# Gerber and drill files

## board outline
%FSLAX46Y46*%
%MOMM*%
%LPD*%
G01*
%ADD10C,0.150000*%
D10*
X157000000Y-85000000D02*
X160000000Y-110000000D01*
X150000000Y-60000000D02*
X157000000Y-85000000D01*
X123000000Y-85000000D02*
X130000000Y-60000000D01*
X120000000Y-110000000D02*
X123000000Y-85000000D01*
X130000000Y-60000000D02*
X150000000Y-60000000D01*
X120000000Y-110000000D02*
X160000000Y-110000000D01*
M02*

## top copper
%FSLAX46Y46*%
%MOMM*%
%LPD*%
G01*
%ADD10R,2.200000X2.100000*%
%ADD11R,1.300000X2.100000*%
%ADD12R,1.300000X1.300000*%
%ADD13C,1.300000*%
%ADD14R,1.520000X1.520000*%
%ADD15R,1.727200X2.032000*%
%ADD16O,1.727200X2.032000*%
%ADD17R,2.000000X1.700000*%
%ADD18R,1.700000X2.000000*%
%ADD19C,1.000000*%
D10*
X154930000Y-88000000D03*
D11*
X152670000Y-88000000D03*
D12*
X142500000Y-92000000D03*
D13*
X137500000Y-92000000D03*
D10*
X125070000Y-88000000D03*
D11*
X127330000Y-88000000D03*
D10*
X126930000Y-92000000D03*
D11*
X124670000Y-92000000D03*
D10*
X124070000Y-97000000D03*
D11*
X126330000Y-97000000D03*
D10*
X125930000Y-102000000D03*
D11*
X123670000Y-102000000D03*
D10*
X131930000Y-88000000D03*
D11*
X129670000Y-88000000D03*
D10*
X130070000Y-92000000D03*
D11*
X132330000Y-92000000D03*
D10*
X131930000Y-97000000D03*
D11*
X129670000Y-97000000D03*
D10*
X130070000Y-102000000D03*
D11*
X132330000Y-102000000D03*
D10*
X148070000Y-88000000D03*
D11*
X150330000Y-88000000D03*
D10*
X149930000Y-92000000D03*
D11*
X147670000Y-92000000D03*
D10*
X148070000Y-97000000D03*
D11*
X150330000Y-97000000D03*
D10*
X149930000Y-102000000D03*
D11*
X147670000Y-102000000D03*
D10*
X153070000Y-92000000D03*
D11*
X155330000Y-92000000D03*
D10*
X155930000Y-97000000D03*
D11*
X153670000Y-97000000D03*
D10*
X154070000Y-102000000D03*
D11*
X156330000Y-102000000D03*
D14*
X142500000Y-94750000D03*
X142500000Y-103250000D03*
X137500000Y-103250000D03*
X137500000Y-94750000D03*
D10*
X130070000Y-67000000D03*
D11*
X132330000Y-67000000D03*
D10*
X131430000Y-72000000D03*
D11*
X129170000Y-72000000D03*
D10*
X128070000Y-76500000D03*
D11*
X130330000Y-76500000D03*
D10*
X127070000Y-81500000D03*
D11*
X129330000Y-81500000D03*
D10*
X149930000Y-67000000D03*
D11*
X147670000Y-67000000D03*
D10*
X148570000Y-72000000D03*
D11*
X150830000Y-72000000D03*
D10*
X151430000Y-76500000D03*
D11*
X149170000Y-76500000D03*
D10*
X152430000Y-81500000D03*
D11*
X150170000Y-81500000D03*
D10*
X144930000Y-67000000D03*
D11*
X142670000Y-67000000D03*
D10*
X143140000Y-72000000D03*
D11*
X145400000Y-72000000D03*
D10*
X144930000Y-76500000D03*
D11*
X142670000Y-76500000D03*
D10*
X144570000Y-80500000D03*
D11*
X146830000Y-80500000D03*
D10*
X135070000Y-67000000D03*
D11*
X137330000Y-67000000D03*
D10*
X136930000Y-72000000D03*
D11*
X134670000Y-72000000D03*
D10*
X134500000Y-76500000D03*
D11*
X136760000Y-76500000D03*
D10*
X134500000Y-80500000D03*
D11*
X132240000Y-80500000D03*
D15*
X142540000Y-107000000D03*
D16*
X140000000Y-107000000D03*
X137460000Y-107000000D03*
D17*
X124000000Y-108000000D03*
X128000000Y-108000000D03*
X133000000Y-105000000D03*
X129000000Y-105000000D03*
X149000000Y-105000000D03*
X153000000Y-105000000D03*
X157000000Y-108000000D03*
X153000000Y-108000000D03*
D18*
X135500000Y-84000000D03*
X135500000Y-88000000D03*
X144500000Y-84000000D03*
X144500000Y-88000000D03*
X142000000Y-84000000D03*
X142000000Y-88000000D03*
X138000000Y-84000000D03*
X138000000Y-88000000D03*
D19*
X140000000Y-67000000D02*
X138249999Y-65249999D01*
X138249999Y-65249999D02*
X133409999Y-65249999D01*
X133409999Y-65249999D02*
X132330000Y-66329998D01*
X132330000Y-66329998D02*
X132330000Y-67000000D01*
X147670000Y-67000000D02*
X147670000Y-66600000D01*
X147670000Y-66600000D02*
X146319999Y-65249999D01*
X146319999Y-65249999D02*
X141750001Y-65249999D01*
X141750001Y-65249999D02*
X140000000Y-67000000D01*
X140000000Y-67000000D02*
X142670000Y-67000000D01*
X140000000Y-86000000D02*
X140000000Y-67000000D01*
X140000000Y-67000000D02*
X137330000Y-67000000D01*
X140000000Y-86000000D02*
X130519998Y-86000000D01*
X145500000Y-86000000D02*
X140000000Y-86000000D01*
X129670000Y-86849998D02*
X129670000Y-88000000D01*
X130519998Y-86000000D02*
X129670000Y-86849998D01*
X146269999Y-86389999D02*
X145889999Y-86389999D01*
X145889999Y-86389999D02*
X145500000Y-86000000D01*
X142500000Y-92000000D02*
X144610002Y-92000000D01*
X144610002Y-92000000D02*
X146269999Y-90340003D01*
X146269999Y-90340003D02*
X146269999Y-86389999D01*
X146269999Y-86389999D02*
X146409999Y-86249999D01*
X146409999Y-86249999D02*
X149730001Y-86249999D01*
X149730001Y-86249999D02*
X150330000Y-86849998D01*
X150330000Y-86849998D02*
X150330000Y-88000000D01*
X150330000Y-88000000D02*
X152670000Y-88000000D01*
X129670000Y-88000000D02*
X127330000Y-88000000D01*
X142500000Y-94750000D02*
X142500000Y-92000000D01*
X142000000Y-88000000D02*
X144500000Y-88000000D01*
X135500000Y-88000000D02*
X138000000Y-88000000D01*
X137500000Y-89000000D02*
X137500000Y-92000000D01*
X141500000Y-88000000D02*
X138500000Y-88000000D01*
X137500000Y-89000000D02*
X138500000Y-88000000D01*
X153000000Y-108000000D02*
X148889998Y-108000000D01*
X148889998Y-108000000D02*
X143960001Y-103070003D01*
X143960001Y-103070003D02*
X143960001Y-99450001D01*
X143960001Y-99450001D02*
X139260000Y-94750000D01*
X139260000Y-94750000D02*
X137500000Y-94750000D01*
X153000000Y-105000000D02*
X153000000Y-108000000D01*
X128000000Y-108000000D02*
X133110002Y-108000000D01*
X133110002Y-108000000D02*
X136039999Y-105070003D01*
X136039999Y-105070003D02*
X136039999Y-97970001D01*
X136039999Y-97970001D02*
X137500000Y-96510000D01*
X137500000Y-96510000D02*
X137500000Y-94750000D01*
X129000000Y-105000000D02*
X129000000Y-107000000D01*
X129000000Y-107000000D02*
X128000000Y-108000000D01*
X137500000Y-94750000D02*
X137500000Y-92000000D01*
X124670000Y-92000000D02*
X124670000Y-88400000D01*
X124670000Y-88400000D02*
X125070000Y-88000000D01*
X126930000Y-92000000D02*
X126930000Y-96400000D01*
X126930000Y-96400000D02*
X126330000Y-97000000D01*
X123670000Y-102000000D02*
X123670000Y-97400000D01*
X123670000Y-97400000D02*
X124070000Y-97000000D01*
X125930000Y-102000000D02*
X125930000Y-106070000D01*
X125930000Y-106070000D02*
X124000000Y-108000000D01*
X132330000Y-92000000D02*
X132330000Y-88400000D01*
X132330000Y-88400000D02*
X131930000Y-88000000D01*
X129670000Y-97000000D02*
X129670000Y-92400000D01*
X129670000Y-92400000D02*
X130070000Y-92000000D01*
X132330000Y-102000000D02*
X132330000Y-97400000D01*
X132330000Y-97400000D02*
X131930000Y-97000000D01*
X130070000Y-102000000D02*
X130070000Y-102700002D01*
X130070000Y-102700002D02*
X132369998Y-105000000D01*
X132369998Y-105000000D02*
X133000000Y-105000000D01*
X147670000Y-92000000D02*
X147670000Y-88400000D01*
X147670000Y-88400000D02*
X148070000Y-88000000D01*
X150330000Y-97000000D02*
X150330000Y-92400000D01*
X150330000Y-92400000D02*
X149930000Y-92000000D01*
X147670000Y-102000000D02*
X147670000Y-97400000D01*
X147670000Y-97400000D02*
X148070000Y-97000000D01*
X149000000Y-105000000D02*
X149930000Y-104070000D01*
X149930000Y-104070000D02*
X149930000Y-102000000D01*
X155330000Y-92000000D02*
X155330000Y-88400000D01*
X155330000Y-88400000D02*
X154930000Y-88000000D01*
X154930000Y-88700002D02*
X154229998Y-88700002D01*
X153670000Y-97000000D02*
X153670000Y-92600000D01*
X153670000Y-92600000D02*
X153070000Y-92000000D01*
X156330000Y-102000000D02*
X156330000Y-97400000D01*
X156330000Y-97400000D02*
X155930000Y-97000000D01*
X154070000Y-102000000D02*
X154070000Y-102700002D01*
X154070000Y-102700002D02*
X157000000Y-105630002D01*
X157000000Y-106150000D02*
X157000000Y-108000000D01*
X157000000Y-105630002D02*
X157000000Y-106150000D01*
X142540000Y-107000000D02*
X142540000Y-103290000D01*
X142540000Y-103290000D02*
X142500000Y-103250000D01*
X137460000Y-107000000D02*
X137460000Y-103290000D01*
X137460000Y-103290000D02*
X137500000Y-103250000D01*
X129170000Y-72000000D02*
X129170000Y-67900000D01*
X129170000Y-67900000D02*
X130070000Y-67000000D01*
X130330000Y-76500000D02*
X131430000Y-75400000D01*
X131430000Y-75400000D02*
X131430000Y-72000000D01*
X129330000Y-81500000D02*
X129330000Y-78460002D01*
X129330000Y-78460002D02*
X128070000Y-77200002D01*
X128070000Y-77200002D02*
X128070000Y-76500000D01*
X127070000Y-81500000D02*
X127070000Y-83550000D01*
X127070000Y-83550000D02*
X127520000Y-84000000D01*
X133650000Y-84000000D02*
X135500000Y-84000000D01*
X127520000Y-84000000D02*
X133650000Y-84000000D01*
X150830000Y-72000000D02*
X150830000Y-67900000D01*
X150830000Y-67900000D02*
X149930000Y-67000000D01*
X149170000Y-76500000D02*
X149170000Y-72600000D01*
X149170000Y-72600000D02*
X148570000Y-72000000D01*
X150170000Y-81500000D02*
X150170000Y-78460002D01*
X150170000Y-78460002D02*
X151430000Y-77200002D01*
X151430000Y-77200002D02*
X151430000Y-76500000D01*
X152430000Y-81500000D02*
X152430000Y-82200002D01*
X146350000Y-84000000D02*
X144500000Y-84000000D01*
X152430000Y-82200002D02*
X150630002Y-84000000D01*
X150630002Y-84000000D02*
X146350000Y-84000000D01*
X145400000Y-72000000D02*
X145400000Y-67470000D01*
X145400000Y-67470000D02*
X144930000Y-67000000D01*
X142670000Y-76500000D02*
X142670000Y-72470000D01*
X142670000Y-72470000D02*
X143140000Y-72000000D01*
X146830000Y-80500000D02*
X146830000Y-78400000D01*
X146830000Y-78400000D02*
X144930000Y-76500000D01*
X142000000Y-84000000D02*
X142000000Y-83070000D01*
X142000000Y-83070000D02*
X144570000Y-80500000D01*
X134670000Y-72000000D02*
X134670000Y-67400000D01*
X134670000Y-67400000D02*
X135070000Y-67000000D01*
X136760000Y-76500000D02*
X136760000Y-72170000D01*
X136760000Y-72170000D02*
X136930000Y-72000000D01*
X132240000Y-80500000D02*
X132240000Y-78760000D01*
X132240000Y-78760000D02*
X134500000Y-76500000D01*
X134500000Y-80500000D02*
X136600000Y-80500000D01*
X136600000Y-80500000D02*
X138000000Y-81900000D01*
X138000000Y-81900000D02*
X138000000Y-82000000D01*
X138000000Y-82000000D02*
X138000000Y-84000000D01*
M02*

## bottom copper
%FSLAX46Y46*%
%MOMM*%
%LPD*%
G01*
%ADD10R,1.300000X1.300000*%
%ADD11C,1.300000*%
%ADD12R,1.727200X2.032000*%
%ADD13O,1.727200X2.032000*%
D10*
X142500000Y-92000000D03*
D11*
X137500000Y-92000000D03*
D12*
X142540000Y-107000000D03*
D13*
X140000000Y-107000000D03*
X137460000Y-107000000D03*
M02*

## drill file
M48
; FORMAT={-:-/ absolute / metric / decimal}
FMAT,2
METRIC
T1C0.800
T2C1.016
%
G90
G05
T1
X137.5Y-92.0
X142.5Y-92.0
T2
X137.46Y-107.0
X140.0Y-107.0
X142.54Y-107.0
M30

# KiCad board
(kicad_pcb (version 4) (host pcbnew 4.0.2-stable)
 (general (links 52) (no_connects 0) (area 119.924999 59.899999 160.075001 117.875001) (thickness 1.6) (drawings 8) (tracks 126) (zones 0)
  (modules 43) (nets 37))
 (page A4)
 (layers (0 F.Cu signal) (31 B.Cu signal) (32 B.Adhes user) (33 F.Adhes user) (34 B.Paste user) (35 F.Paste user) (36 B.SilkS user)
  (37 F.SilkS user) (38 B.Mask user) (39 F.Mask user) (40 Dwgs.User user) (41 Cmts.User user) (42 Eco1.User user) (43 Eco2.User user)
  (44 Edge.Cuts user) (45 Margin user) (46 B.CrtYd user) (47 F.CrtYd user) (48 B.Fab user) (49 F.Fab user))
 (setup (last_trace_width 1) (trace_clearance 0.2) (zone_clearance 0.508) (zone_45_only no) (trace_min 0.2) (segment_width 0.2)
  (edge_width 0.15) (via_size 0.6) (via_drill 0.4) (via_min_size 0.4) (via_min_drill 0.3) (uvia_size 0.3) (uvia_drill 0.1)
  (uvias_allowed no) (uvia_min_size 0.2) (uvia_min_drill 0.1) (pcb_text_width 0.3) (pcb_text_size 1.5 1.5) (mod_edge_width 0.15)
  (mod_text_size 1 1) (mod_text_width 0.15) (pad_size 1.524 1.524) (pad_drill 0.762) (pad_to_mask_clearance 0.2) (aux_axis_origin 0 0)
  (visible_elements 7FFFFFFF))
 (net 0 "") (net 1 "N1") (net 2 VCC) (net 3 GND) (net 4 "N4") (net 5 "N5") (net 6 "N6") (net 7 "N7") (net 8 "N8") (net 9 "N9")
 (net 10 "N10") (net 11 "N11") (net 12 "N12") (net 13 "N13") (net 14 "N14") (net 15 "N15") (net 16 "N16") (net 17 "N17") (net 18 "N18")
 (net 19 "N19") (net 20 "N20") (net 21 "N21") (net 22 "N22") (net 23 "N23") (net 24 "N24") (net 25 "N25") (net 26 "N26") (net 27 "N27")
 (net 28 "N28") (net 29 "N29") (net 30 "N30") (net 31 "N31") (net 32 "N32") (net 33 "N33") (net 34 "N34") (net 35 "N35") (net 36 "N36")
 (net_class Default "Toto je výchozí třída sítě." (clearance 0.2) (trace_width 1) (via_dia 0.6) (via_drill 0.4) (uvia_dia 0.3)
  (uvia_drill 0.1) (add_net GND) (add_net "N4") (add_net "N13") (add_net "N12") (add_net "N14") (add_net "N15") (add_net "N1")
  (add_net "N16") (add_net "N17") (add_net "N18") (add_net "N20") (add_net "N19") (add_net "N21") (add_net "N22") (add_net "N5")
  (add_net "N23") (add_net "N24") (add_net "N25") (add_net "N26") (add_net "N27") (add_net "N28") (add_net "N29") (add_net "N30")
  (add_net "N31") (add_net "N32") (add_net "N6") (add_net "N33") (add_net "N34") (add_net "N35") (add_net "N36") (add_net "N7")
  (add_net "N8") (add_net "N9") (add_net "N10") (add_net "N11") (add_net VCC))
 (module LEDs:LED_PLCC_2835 (layer F.Cu) (at 154 88)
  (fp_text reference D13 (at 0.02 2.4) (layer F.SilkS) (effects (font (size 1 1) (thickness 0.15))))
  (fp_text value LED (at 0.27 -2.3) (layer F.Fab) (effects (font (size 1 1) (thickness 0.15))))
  (pad 1 smd rect (at 0.93 0) (size 2.2 2.1) (layers F.Cu F.Paste F.Mask) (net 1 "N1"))
  (pad 2 smd rect (at -1.33 0) (size 1.3 2.1) (layers F.Cu F.Paste F.Mask) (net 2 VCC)))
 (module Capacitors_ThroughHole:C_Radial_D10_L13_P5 (layer F.Cu) (at 142.5 92 180)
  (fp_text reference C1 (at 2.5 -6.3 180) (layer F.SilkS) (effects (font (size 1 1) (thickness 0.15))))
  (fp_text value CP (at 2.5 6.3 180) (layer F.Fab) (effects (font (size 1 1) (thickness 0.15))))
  (pad 1 thru_hole rect (at 0 0 180) (size 1.3 1.3) (drill 0.8) (layers *.Cu *.Mask F.SilkS) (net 2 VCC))
  (pad 2 thru_hole circle (at 5 0 180) (size 1.3 1.3) (drill 0.8) (layers *.Cu *.Mask F.SilkS) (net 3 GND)))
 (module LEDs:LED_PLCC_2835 (layer F.Cu) (at 126 88 180)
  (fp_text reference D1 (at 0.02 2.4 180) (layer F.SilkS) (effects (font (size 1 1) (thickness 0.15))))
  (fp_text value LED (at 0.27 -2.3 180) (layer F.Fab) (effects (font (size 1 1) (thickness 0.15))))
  (pad 1 smd rect (at 0.93 0 180) (size 2.2 2.1) (layers F.Cu F.Paste F.Mask) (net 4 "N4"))
  (pad 2 smd rect (at -1.33 0 180) (size 1.3 2.1) (layers F.Cu F.Paste F.Mask) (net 2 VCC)))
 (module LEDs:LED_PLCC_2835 (layer F.Cu) (at 126 92)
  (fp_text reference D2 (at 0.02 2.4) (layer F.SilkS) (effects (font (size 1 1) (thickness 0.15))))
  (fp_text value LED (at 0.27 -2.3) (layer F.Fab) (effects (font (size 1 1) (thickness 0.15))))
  (pad 1 smd rect (at 0.93 0) (size 2.2 2.1) (layers F.Cu F.Paste F.Mask) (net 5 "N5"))
  (pad 2 smd rect (at -1.33 0) (size 1.3 2.1) (layers F.Cu F.Paste F.Mask) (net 4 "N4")))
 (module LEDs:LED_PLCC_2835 (layer F.Cu) (at 125 97 180)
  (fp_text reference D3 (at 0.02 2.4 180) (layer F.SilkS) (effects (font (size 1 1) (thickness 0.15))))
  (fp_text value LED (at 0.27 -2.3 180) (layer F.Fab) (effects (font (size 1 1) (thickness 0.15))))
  (pad 1 smd rect (at 0.93 0 180) (size 2.2 2.1) (layers F.Cu F.Paste F.Mask) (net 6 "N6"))
  (pad 2 smd rect (at -1.33 0 180) (size 1.3 2.1) (layers F.Cu F.Paste F.Mask) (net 5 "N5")))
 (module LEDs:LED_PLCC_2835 (layer F.Cu) (at 125 102)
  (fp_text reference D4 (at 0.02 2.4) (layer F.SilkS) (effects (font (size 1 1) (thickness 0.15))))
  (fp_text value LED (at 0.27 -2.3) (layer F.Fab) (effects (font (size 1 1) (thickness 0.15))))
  (pad 1 smd rect (at 0.93 0) (size 2.2 2.1) (layers F.Cu F.Paste F.Mask) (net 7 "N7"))
  (pad 2 smd rect (at -1.33 0) (size 1.3 2.1) (layers F.Cu F.Paste F.Mask) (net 6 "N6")))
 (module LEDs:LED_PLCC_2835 (layer F.Cu) (at 131 88)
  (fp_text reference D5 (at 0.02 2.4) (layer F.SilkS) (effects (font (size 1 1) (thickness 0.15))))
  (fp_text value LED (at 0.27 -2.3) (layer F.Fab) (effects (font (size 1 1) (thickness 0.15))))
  (pad 1 smd rect (at 0.93 0) (size 2.2 2.1) (layers F.Cu F.Paste F.Mask) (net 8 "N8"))
  (pad 2 smd rect (at -1.33 0) (size 1.3 2.1) (layers F.Cu F.Paste F.Mask) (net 2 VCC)))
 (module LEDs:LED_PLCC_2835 (layer F.Cu) (at 131 92 180)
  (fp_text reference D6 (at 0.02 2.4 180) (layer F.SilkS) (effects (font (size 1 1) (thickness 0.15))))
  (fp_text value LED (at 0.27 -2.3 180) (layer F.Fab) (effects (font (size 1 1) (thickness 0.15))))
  (pad 1 smd rect (at 0.93 0 180) (size 2.2 2.1) (layers F.Cu F.Paste F.Mask) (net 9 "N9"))
  (pad 2 smd rect (at -1.33 0 180) (size 1.3 2.1) (layers F.Cu F.Paste F.Mask) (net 8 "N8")))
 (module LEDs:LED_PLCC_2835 (layer F.Cu) (at 131 97)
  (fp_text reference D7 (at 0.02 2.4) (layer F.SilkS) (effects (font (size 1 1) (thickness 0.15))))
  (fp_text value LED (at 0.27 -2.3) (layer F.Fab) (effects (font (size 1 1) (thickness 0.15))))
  (pad 1 smd rect (at 0.93 0) (size 2.2 2.1) (layers F.Cu F.Paste F.Mask) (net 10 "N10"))
  (pad 2 smd rect (at -1.33 0) (size 1.3 2.1) (layers F.Cu F.Paste F.Mask) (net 9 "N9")))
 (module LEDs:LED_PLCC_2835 (layer F.Cu) (at 131 102 180)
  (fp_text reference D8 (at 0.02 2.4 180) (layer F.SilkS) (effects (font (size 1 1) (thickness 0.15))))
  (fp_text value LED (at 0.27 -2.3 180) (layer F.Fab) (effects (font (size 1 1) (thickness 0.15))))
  (pad 1 smd rect (at 0.93 0 180) (size 2.2 2.1) (layers F.Cu F.Paste F.Mask) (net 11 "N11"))
  (pad 2 smd rect (at -1.33 0 180) (size 1.3 2.1) (layers F.Cu F.Paste F.Mask) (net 10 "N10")))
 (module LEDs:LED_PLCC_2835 (layer F.Cu) (at 149 88 180)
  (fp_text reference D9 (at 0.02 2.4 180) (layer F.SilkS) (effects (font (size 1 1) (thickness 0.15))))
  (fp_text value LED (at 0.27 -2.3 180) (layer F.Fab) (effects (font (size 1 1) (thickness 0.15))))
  (pad 1 smd rect (at 0.93 0 180) (size 2.2 2.1) (layers F.Cu F.Paste F.Mask) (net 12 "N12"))
  (pad 2 smd rect (at -1.33 0 180) (size 1.3 2.1) (layers F.Cu F.Paste F.Mask) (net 2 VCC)))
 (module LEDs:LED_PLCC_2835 (layer F.Cu) (at 149 92)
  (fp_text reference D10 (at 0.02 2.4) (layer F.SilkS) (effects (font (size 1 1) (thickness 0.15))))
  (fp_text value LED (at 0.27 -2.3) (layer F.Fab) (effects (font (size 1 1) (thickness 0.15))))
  (pad 1 smd rect (at 0.93 0) (size 2.2 2.1) (layers F.Cu F.Paste F.Mask) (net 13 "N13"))
  (pad 2 smd rect (at -1.33 0) (size 1.3 2.1) (layers F.Cu F.Paste F.Mask) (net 12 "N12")))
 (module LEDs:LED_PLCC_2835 (layer F.Cu) (at 149 97 180)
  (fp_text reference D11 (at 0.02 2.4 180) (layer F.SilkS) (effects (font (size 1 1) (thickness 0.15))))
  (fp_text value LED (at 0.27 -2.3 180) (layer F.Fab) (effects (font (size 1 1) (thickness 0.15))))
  (pad 1 smd rect (at 0.93 0 180) (size 2.2 2.1) (layers F.Cu F.Paste F.Mask) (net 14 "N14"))
  (pad 2 smd rect (at -1.33 0 180) (size 1.3 2.1) (layers F.Cu F.Paste F.Mask) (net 13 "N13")))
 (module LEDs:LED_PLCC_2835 (layer F.Cu) (at 149 102)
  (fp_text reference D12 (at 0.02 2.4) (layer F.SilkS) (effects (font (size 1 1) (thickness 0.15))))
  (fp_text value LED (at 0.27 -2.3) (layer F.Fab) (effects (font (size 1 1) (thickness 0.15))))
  (pad 1 smd rect (at 0.93 0) (size 2.2 2.1) (layers F.Cu F.Paste F.Mask) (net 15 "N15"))
  (pad 2 smd rect (at -1.33 0) (size 1.3 2.1) (layers F.Cu F.Paste F.Mask) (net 14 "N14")))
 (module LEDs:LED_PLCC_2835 (layer F.Cu) (at 154 92 180)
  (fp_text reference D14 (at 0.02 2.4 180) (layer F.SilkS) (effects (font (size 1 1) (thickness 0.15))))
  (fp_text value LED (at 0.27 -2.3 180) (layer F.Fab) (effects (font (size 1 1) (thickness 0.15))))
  (pad 1 smd rect (at 0.93 0 180) (size 2.2 2.1) (layers F.Cu F.Paste F.Mask) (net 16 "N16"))
  (pad 2 smd rect (at -1.33 0 180) (size 1.3 2.1) (layers F.Cu F.Paste F.Mask) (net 1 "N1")))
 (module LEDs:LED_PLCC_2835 (layer F.Cu) (at 155 97)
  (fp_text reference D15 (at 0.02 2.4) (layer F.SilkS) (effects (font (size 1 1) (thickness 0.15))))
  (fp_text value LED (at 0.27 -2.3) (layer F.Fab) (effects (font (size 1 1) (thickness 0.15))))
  (pad 1 smd rect (at 0.93 0) (size 2.2 2.1) (layers F.Cu F.Paste F.Mask) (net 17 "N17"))
  (pad 2 smd rect (at -1.33 0) (size 1.3 2.1) (layers F.Cu F.Paste F.Mask) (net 16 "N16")))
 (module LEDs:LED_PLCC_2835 (layer F.Cu) (at 155 102 180)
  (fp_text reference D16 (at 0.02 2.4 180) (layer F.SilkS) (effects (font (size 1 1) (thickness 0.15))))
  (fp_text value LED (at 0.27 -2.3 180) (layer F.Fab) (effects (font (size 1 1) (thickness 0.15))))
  (pad 1 smd rect (at 0.93 0 180) (size 2.2 2.1) (layers F.Cu F.Paste F.Mask) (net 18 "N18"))
  (pad 2 smd rect (at -1.33 0 180) (size 1.3 2.1) (layers F.Cu F.Paste F.Mask) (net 17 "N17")))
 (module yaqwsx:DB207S (layer F.Cu) (at 140 99)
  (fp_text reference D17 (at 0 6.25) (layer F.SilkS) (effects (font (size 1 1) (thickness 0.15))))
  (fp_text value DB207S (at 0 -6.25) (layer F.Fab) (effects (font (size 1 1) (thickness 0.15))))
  (pad 3 smd rect (at 2.5 -4.25) (size 1.52 1.52) (layers F.Cu F.Paste F.Mask) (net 2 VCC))
  (pad 4 smd rect (at 2.5 4.25) (size 1.52 1.52) (layers F.Cu F.Paste F.Mask) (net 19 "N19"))
  (pad 2 smd rect (at -2.5 4.25) (size 1.52 1.52) (layers F.Cu F.Paste F.Mask) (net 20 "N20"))
  (pad 1 smd rect (at -2.5 -4.25) (size 1.52 1.52) (layers F.Cu F.Paste F.Mask) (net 3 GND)))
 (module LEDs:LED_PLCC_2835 (layer F.Cu) (at 131 67 180)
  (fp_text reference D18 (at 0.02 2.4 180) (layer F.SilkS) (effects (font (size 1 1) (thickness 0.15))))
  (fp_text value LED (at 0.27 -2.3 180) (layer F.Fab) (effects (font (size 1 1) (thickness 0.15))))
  (pad 1 smd rect (at 0.93 0 180) (size 2.2 2.1) (layers F.Cu F.Paste F.Mask) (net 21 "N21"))
  (pad 2 smd rect (at -1.33 0 180) (size 1.3 2.1) (layers F.Cu F.Paste F.Mask) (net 2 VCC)))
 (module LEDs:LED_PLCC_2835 (layer F.Cu) (at 130.5 72)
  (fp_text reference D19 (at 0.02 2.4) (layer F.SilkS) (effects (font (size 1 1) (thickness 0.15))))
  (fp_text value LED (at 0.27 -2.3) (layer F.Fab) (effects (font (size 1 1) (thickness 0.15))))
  (pad 1 smd rect (at 0.93 0) (size 2.2 2.1) (layers F.Cu F.Paste F.Mask) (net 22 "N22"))
  (pad 2 smd rect (at -1.33 0) (size 1.3 2.1) (layers F.Cu F.Paste F.Mask) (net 21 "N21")))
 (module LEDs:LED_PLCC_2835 (layer F.Cu) (at 129 76.5 180)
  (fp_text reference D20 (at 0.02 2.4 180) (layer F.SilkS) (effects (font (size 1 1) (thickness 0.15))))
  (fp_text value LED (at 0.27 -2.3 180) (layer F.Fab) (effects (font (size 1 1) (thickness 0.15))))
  (pad 1 smd rect (at 0.93 0 180) (size 2.2 2.1) (layers F.Cu F.Paste F.Mask) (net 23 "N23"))
  (pad 2 smd rect (at -1.33 0 180) (size 1.3 2.1) (layers F.Cu F.Paste F.Mask) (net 22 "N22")))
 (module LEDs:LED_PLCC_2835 (layer F.Cu) (at 128 81.5 180)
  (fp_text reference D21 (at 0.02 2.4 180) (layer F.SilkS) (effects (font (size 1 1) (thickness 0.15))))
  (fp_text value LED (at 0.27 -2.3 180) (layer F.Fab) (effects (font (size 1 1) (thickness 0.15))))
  (pad 1 smd rect (at 0.93 0 180) (size 2.2 2.1) (layers F.Cu F.Paste F.Mask) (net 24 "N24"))
  (pad 2 smd rect (at -1.33 0 180) (size 1.3 2.1) (layers F.Cu F.Paste F.Mask) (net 23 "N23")))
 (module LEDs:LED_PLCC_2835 (layer F.Cu) (at 149 67)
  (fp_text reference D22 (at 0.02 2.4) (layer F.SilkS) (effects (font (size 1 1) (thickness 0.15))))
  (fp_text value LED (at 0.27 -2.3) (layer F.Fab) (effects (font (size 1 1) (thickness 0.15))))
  (pad 1 smd rect (at 0.93 0) (size 2.2 2.1) (layers F.Cu F.Paste F.Mask) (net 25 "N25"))
  (pad 2 smd rect (at -1.33 0) (size 1.3 2.1) (layers F.Cu F.Paste F.Mask) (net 2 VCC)))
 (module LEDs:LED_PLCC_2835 (layer F.Cu) (at 149.5 72 180)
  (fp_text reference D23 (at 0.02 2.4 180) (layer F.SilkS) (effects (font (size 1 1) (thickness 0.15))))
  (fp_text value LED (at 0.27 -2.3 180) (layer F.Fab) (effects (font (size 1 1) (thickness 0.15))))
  (pad 1 smd rect (at 0.93 0 180) (size 2.2 2.1) (layers F.Cu F.Paste F.Mask) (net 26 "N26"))
  (pad 2 smd rect (at -1.33 0 180) (size 1.3 2.1) (layers F.Cu F.Paste F.Mask) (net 25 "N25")))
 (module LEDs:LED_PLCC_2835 (layer F.Cu) (at 150.5 76.5)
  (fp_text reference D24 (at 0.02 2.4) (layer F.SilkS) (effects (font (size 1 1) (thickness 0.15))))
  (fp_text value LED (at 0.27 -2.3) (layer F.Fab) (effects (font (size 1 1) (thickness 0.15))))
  (pad 1 smd rect (at 0.93 0) (size 2.2 2.1) (layers F.Cu F.Paste F.Mask) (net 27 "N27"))
  (pad 2 smd rect (at -1.33 0) (size 1.3 2.1) (layers F.Cu F.Paste F.Mask) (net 26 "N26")))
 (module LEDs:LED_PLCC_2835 (layer F.Cu) (at 151.5 81.5)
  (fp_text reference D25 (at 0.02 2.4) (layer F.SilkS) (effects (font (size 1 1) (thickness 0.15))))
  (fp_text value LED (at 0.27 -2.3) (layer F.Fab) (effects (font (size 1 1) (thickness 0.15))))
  (pad 1 smd rect (at 0.93 0) (size 2.2 2.1) (layers F.Cu F.Paste F.Mask) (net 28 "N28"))
  (pad 2 smd rect (at -1.33 0) (size 1.3 2.1) (layers F.Cu F.Paste F.Mask) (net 27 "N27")))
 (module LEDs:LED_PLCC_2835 (layer F.Cu) (at 144 67)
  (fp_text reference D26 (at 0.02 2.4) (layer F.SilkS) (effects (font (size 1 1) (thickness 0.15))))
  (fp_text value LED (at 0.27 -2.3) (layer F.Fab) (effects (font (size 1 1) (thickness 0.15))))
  (pad 1 smd rect (at 0.93 0) (size 2.2 2.1) (layers F.Cu F.Paste F.Mask) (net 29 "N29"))
  (pad 2 smd rect (at -1.33 0) (size 1.3 2.1) (layers F.Cu F.Paste F.Mask) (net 2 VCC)))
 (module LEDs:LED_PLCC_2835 (layer F.Cu) (at 144.07 72 180)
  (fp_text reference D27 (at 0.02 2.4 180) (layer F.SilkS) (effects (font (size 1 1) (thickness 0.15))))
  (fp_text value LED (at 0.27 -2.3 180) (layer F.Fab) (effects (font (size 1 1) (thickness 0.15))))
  (pad 1 smd rect (at 0.93 0 180) (size 2.2 2.1) (layers F.Cu F.Paste F.Mask) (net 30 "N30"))
  (pad 2 smd rect (at -1.33 0 180) (size 1.3 2.1) (layers F.Cu F.Paste F.Mask) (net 29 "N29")))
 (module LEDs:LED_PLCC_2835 (layer F.Cu) (at 144 76.5)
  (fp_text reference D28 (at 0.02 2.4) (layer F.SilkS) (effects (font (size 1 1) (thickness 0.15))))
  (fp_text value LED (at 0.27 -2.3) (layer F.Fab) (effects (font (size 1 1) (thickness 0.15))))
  (pad 1 smd rect (at 0.93 0) (size 2.2 2.1) (layers F.Cu F.Paste F.Mask) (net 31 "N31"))
  (pad 2 smd rect (at -1.33 0) (size 1.3 2.1) (layers F.Cu F.Paste F.Mask) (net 30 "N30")))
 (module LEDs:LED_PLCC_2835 (layer F.Cu) (at 145.5 80.5 180)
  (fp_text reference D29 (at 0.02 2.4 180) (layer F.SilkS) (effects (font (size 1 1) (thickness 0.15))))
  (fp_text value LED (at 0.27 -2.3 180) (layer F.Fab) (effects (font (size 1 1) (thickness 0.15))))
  (pad 1 smd rect (at 0.93 0 180) (size 2.2 2.1) (layers F.Cu F.Paste F.Mask) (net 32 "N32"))
  (pad 2 smd rect (at -1.33 0 180) (size 1.3 2.1) (layers F.Cu F.Paste F.Mask) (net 31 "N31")))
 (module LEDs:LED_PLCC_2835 (layer F.Cu) (at 136 67 180)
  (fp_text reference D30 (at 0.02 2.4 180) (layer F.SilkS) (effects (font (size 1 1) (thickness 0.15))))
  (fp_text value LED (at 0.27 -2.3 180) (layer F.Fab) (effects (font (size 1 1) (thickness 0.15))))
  (pad 1 smd rect (at 0.93 0 180) (size 2.2 2.1) (layers F.Cu F.Paste F.Mask) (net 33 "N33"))
  (pad 2 smd rect (at -1.33 0 180) (size 1.3 2.1) (layers F.Cu F.Paste F.Mask) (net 2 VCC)))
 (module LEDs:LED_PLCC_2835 (layer F.Cu) (at 136 72)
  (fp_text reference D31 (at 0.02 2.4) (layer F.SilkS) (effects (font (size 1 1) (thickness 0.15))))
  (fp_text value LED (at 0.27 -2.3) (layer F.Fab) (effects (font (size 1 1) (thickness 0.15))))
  (pad 1 smd rect (at 0.93 0) (size 2.2 2.1) (layers F.Cu F.Paste F.Mask) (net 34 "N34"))
  (pad 2 smd rect (at -1.33 0) (size 1.3 2.1) (layers F.Cu F.Paste F.Mask) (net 33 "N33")))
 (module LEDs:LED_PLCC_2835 (layer F.Cu) (at 135.43 76.5 180)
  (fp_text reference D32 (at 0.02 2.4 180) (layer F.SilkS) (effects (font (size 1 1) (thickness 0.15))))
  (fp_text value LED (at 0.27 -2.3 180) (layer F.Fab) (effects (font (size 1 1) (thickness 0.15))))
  (pad 1 smd rect (at 0.93 0 180) (size 2.2 2.1) (layers F.Cu F.Paste F.Mask) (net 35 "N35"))
  (pad 2 smd rect (at -1.33 0 180) (size 1.3 2.1) (layers F.Cu F.Paste F.Mask) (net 34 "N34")))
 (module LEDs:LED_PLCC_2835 (layer F.Cu) (at 133.57 80.5)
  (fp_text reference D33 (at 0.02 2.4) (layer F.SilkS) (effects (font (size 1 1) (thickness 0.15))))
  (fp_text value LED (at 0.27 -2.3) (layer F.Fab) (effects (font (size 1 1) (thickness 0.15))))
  (pad 1 smd rect (at 0.93 0) (size 2.2 2.1) (layers F.Cu F.Paste F.Mask) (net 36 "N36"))
  (pad 2 smd rect (at -1.33 0) (size 1.3 2.1) (layers F.Cu F.Paste F.Mask) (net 35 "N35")))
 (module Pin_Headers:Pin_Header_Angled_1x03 (layer F.Cu) (at 142.54 107 270)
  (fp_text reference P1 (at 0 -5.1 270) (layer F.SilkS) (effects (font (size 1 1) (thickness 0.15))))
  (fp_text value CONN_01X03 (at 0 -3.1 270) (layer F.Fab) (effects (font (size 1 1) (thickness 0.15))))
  (pad 1 thru_hole rect (at 0 0 270) (size 2.032 1.7272) (drill 1.016) (layers *.Cu *.Mask F.SilkS) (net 19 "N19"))
  (pad 2 thru_hole oval (at 0 2.54 270) (size 2.032 1.7272) (drill 1.016) (layers *.Cu *.Mask F.SilkS))
  (pad 3 thru_hole oval (at 0 5.08 270) (size 2.032 1.7272) (drill 1.016) (layers *.Cu *.Mask F.SilkS) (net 20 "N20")))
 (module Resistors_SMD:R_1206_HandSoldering (layer F.Cu) (at 126 108)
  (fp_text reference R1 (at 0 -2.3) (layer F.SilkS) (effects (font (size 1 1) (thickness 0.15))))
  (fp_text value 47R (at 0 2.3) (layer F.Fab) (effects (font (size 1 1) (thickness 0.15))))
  (pad 1 smd rect (at -2 0) (size 2 1.7) (layers F.Cu F.Paste F.Mask) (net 7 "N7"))
  (pad 2 smd rect (at 2 0) (size 2 1.7) (layers F.Cu F.Paste F.Mask) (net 3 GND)))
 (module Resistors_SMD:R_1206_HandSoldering (layer F.Cu) (at 131 105 180)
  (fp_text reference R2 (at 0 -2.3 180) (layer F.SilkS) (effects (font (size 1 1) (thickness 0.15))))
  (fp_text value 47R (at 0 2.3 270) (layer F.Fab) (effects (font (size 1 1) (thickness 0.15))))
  (pad 1 smd rect (at -2 0 180) (size 2 1.7) (layers F.Cu F.Paste F.Mask) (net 11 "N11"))
  (pad 2 smd rect (at 2 0 180) (size 2 1.7) (layers F.Cu F.Paste F.Mask) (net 3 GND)))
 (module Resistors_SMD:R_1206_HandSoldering (layer F.Cu) (at 151 105)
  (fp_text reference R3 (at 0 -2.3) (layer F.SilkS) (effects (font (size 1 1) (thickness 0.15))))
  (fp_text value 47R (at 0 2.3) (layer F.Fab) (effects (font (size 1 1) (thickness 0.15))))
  (pad 1 smd rect (at -2 0) (size 2 1.7) (layers F.Cu F.Paste F.Mask) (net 15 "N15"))
  (pad 2 smd rect (at 2 0) (size 2 1.7) (layers F.Cu F.Paste F.Mask) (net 3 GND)))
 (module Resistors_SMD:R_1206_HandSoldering (layer F.Cu) (at 155 108 180)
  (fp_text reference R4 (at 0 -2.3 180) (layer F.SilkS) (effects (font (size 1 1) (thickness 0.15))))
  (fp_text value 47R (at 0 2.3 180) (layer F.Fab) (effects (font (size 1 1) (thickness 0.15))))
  (pad 1 smd rect (at -2 0 180) (size 2 1.7) (layers F.Cu F.Paste F.Mask) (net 18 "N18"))
  (pad 2 smd rect (at 2 0 180) (size 2 1.7) (layers F.Cu F.Paste F.Mask) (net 3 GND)))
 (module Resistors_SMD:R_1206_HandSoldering (layer F.Cu) (at 135.5 86 270)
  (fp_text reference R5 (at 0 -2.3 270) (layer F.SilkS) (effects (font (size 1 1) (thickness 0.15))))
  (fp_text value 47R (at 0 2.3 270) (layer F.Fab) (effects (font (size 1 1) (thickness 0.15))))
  (pad 1 smd rect (at -2 0 270) (size 2 1.7) (layers F.Cu F.Paste F.Mask) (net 24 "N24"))
  (pad 2 smd rect (at 2 0 270) (size 2 1.7) (layers F.Cu F.Paste F.Mask) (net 3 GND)))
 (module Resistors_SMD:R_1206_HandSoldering (layer F.Cu) (at 144.5 86 270)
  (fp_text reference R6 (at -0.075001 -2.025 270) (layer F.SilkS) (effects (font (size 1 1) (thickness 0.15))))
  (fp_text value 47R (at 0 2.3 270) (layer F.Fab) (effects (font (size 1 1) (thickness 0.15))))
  (pad 1 smd rect (at -2 0 270) (size 2 1.7) (layers F.Cu F.Paste F.Mask) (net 28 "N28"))
  (pad 2 smd rect (at 2 0 270) (size 2 1.7) (layers F.Cu F.Paste F.Mask) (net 3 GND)))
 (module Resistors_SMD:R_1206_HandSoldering (layer F.Cu) (at 142 86 270)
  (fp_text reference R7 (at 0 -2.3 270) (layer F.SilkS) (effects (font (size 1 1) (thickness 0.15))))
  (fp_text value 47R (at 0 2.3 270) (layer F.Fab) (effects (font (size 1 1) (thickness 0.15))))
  (pad 1 smd rect (at -2 0 270) (size 2 1.7) (layers F.Cu F.Paste F.Mask) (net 32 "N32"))
  (pad 2 smd rect (at 2 0 270) (size 2 1.7) (layers F.Cu F.Paste F.Mask) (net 3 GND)))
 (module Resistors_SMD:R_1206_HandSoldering (layer F.Cu) (at 138 86 270)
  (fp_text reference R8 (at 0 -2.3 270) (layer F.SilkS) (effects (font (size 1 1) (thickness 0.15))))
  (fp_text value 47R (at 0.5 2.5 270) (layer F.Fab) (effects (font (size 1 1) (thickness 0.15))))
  (pad 1 smd rect (at -2 0 270) (size 2 1.7) (layers F.Cu F.Paste F.Mask) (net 36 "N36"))
  (pad 2 smd rect (at 2 0 270) (size 2 1.7) (layers F.Cu F.Paste F.Mask) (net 3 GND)))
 (gr_line (start 157 85) (end 160 110) (layer Edge.Cuts) (width 0.15))
 (gr_line (start 150 60) (end 157 85) (layer Edge.Cuts) (width 0.15))
 (gr_line (start 123 85) (end 130 60) (layer Edge.Cuts) (width 0.15))
 (gr_line (start 120 110) (end 123 85) (layer Edge.Cuts) (width 0.15))
 (gr_line (start 130 60) (end 150 60) (layer Edge.Cuts) (width 0.15))
 (gr_line (start 120 110) (end 160 110) (layer Edge.Cuts) (width 0.15))
 (segment (start 140 67) (end 138.249999 65.249999) (width 1) (layer F.Cu) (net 2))
 (segment (start 138.249999 65.249999) (end 133.409999 65.249999) (width 1) (layer F.Cu) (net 2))
 (segment (start 133.409999 65.249999) (end 132.33 66.329998) (width 1) (layer F.Cu) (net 2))
 (segment (start 132.33 66.329998) (end 132.33 67) (width 1) (layer F.Cu) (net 2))
 (segment (start 147.67 67) (end 147.67 66.6) (width 1) (layer F.Cu) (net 2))
 (segment (start 147.67 66.6) (end 146.319999 65.249999) (width 1) (layer F.Cu) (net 2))
 (segment (start 146.319999 65.249999) (end 141.750001 65.249999) (width 1) (layer F.Cu) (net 2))
 (segment (start 141.750001 65.249999) (end 140 67) (width 1) (layer F.Cu) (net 2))
 (segment (start 140 67) (end 142.67 67) (width 1) (layer F.Cu) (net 2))
 (segment (start 140 86) (end 140 67) (width 1) (layer F.Cu) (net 2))
 (segment (start 140 67) (end 137.33 67) (width 1) (layer F.Cu) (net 2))
 (segment (start 140 86) (end 130.519998 86) (width 1) (layer F.Cu) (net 2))
 (segment (start 145.5 86) (end 140 86) (width 1) (layer F.Cu) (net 2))
 (segment (start 129.67 86.849998) (end 129.67 88) (width 1) (layer F.Cu) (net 2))
 (segment (start 130.519998 86) (end 129.67 86.849998) (width 1) (layer F.Cu) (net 2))
 (segment (start 146.269999 86.389999) (end 145.889999 86.389999) (width 1) (layer F.Cu) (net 2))
 (segment (start 145.889999 86.389999) (end 145.5 86) (width 1) (layer F.Cu) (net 2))
 (segment (start 142.5 92) (end 144.610002 92) (width 1) (layer F.Cu) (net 2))
 (segment (start 144.610002 92) (end 146.269999 90.340003) (width 1) (layer F.Cu) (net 2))
 (segment (start 146.269999 90.340003) (end 146.269999 86.389999) (width 1) (layer F.Cu) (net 2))
 (segment (start 146.269999 86.389999) (end 146.409999 86.249999) (width 1) (layer F.Cu) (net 2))
 (segment (start 146.409999 86.249999) (end 149.730001 86.249999) (width 1) (layer F.Cu) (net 2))
 (segment (start 149.730001 86.249999) (end 150.33 86.849998) (width 1) (layer F.Cu) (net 2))
 (segment (start 150.33 86.849998) (end 150.33 88) (width 1) (layer F.Cu) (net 2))
 (segment (start 150.33 88) (end 152.67 88) (width 1) (layer F.Cu) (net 2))
 (segment (start 129.67 88) (end 127.33 88) (width 1) (layer F.Cu) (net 2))
 (segment (start 142.5 94.75) (end 142.5 92) (width 1) (layer F.Cu) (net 2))
 (segment (start 142 88) (end 144.5 88) (width 1) (layer F.Cu) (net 3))
 (segment (start 135.5 88) (end 138 88) (width 1) (layer F.Cu) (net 3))
 (segment (start 137.5 89) (end 137.5 92) (width 1) (layer F.Cu) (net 3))
 (segment (start 141.5 88) (end 138.5 88) (width 1) (layer F.Cu) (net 3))
 (segment (start 137.5 89) (end 138.5 88) (width 1) (layer F.Cu) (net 3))
 (segment (start 153 108) (end 148.889998 108) (width 1) (layer F.Cu) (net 3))
 (segment (start 148.889998 108) (end 143.960001 103.070003) (width 1) (layer F.Cu) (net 3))
 (segment (start 143.960001 103.070003) (end 143.960001 99.450001) (width 1) (layer F.Cu) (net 3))
 (segment (start 143.960001 99.450001) (end 139.26 94.75) (width 1) (layer F.Cu) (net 3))
 (segment (start 139.26 94.75) (end 137.5 94.75) (width 1) (layer F.Cu) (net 3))
 (segment (start 153 105) (end 153 108) (width 1) (layer F.Cu) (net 3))
 (segment (start 128 108) (end 133.110002 108) (width 1) (layer F.Cu) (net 3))
 (segment (start 133.110002 108) (end 136.039999 105.070003) (width 1) (layer F.Cu) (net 3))
 (segment (start 136.039999 105.070003) (end 136.039999 97.970001) (width 1) (layer F.Cu) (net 3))
 (segment (start 136.039999 97.970001) (end 137.5 96.51) (width 1) (layer F.Cu) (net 3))
 (segment (start 137.5 96.51) (end 137.5 94.75) (width 1) (layer F.Cu) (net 3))
 (segment (start 129 105) (end 129 107) (width 1) (layer F.Cu) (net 3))
 (segment (start 129 107) (end 128 108) (width 1) (layer F.Cu) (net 3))
 (segment (start 137.5 94.75) (end 137.5 92) (width 1) (layer F.Cu) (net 3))
 (segment (start 124.67 92) (end 124.67 88.4) (width 1) (layer F.Cu) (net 4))
 (segment (start 124.67 88.4) (end 125.07 88) (width 1) (layer F.Cu) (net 4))
 (segment (start 126.93 92) (end 126.93 96.4) (width 1) (layer F.Cu) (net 5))
 (segment (start 126.93 96.4) (end 126.33 97) (width 1) (layer F.Cu) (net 5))
 (segment (start 123.67 102) (end 123.67 97.4) (width 1) (layer F.Cu) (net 6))
 (segment (start 123.67 97.4) (end 124.07 97) (width 1) (layer F.Cu) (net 6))
 (segment (start 125.93 102) (end 125.93 106.07) (width 1) (layer F.Cu) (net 7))
 (segment (start 125.93 106.07) (end 124 108) (width 1) (layer F.Cu) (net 7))
 (segment (start 132.33 92) (end 132.33 88.4) (width 1) (layer F.Cu) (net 8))
 (segment (start 132.33 88.4) (end 131.93 88) (width 1) (layer F.Cu) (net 8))
 (segment (start 129.67 97) (end 129.67 92.4) (width 1) (layer F.Cu) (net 9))
 (segment (start 129.67 92.4) (end 130.07 92) (width 1) (layer F.Cu) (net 9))
 (segment (start 132.33 102) (end 132.33 97.4) (width 1) (layer F.Cu) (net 10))
 (segment (start 132.33 97.4) (end 131.93 97) (width 1) (layer F.Cu) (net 10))
 (segment (start 130.07 102) (end 130.07 102.700002) (width 1) (layer F.Cu) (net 11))
 (segment (start 130.07 102.700002) (end 132.369998 105) (width 1) (layer F.Cu) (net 11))
 (segment (start 132.369998 105) (end 133 105) (width 1) (layer F.Cu) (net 11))
 (segment (start 147.67 92) (end 147.67 88.4) (width 1) (layer F.Cu) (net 12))
 (segment (start 147.67 88.4) (end 148.07 88) (width 1) (layer F.Cu) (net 12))
 (segment (start 150.33 97) (end 150.33 92.4) (width 1) (layer F.Cu) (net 13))
 (segment (start 150.33 92.4) (end 149.93 92) (width 1) (layer F.Cu) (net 13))
 (segment (start 147.67 102) (end 147.67 97.4) (width 1) (layer F.Cu) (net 14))
 (segment (start 147.67 97.4) (end 148.07 97) (width 1) (layer F.Cu) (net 14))
 (segment (start 149 105) (end 149.93 104.07) (width 1) (layer F.Cu) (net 15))
 (segment (start 149.93 104.07) (end 149.93 102) (width 1) (layer F.Cu) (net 15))
 (segment (start 155.33 92) (end 155.33 88.4) (width 1) (layer F.Cu) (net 1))
 (segment (start 155.33 88.4) (end 154.93 88) (width 1) (layer F.Cu) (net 1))
 (segment (start 154.93 88.700002) (end 154.229998 88.700002) (width 1) (layer F.Cu) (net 1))
 (segment (start 153.67 97) (end 153.67 92.6) (width 1) (layer F.Cu) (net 16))
 (segment (start 153.67 92.6) (end 153.07 92) (width 1) (layer F.Cu) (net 16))
 (segment (start 156.33 102) (end 156.33 97.4) (width 1) (layer F.Cu) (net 17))
 (segment (start 156.33 97.4) (end 155.93 97) (width 1) (layer F.Cu) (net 17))
 (segment (start 154.07 102) (end 154.07 102.700002) (width 1) (layer F.Cu) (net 18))
 (segment (start 154.07 102.700002) (end 157 105.630002) (width 1) (layer F.Cu) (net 18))
 (segment (start 157 106.15) (end 157 108) (width 1) (layer F.Cu) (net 18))
 (segment (start 157 105.630002) (end 157 106.15) (width 1) (layer F.Cu) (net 18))
 (segment (start 142.54 107) (end 142.54 103.29) (width 1) (layer F.Cu) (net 19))
 (segment (start 142.54 103.29) (end 142.5 103.25) (width 1) (layer F.Cu) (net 19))
 (segment (start 137.46 107) (end 137.46 103.29) (width 1) (layer F.Cu) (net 20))
 (segment (start 137.46 103.29) (end 137.5 103.25) (width 1) (layer F.Cu) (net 20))
 (segment (start 129.17 72) (end 129.17 67.9) (width 1) (layer F.Cu) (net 21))
 (segment (start 129.17 67.9) (end 130.07 67) (width 1) (layer F.Cu) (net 21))
 (segment (start 130.33 76.5) (end 131.43 75.4) (width 1) (layer F.Cu) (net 22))
 (segment (start 131.43 75.4) (end 131.43 72) (width 1) (layer F.Cu) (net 22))
 (segment (start 129.33 81.5) (end 129.33 78.460002) (width 1) (layer F.Cu) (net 23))
 (segment (start 129.33 78.460002) (end 128.07 77.200002) (width 1) (layer F.Cu) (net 23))
 (segment (start 128.07 77.200002) (end 128.07 76.5) (width 1) (layer F.Cu) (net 23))
 (segment (start 127.07 81.5) (end 127.07 83.55) (width 1) (layer F.Cu) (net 24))
 (segment (start 127.07 83.55) (end 127.52 84) (width 1) (layer F.Cu) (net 24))
 (segment (start 133.65 84) (end 135.5 84) (width 1) (layer F.Cu) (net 24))
 (segment (start 127.52 84) (end 133.65 84) (width 1) (layer F.Cu) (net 24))
 (segment (start 150.83 72) (end 150.83 67.9) (width 1) (layer F.Cu) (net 25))
 (segment (start 150.83 67.9) (end 149.93 67) (width 1) (layer F.Cu) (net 25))
 (segment (start 149.17 76.5) (end 149.17 72.6) (width 1) (layer F.Cu) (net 26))
 (segment (start 149.17 72.6) (end 148.57 72) (width 1) (layer F.Cu) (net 26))
 (segment (start 150.17 81.5) (end 150.17 78.460002) (width 1) (layer F.Cu) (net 27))
 (segment (start 150.17 78.460002) (end 151.43 77.200002) (width 1) (layer F.Cu) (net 27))
 (segment (start 151.43 77.200002) (end 151.43 76.5) (width 1) (layer F.Cu) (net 27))
 (segment (start 152.43 81.5) (end 152.43 82.200002) (width 1) (layer F.Cu) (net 28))
 (segment (start 146.35 84) (end 144.5 84) (width 1) (layer F.Cu) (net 28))
 (segment (start 152.43 82.200002) (end 150.630002 84) (width 1) (layer F.Cu) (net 28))
 (segment (start 150.630002 84) (end 146.35 84) (width 1) (layer F.Cu) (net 28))
 (segment (start 145.4 72) (end 145.4 67.47) (width 1) (layer F.Cu) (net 29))
 (segment (start 145.4 67.47) (end 144.93 67) (width 1) (layer F.Cu) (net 29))
 (segment (start 142.67 76.5) (end 142.67 72.47) (width 1) (layer F.Cu) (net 30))
 (segment (start 142.67 72.47) (end 143.14 72) (width 1) (layer F.Cu) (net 30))
 (segment (start 146.83 80.5) (end 146.83 78.4) (width 1) (layer F.Cu) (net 31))
 (segment (start 146.83 78.4) (end 144.93 76.5) (width 1) (layer F.Cu) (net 31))
 (segment (start 142 84) (end 142 83.07) (width 1) (layer F.Cu) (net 32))
 (segment (start 142 83.07) (end 144.57 80.5) (width 1) (layer F.Cu) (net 32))
 (segment (start 134.67 72) (end 134.67 67.4) (width 1) (layer F.Cu) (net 33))
 (segment (start 134.67 67.4) (end 135.07 67) (width 1) (layer F.Cu) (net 33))
 (segment (start 136.76 76.5) (end 136.76 72.17) (width 1) (layer F.Cu) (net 34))
 (segment (start 136.76 72.17) (end 136.93 72) (width 1) (layer F.Cu) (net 34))
 (segment (start 132.24 80.5) (end 132.24 78.76) (width 1) (layer F.Cu) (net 35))
 (segment (start 132.24 78.76) (end 134.5 76.5) (width 1) (layer F.Cu) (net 35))
 (segment (start 134.5 80.5) (end 136.6 80.5) (width 1) (layer F.Cu) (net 36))
 (segment (start 136.6 80.5) (end 138 81.9) (width 1) (layer F.Cu) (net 36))
 (segment (start 138 81.9) (end 138 82) (width 1) (layer F.Cu) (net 36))
 (segment (start 138 82) (end 138 84) (width 1) (layer F.Cu) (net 36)))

